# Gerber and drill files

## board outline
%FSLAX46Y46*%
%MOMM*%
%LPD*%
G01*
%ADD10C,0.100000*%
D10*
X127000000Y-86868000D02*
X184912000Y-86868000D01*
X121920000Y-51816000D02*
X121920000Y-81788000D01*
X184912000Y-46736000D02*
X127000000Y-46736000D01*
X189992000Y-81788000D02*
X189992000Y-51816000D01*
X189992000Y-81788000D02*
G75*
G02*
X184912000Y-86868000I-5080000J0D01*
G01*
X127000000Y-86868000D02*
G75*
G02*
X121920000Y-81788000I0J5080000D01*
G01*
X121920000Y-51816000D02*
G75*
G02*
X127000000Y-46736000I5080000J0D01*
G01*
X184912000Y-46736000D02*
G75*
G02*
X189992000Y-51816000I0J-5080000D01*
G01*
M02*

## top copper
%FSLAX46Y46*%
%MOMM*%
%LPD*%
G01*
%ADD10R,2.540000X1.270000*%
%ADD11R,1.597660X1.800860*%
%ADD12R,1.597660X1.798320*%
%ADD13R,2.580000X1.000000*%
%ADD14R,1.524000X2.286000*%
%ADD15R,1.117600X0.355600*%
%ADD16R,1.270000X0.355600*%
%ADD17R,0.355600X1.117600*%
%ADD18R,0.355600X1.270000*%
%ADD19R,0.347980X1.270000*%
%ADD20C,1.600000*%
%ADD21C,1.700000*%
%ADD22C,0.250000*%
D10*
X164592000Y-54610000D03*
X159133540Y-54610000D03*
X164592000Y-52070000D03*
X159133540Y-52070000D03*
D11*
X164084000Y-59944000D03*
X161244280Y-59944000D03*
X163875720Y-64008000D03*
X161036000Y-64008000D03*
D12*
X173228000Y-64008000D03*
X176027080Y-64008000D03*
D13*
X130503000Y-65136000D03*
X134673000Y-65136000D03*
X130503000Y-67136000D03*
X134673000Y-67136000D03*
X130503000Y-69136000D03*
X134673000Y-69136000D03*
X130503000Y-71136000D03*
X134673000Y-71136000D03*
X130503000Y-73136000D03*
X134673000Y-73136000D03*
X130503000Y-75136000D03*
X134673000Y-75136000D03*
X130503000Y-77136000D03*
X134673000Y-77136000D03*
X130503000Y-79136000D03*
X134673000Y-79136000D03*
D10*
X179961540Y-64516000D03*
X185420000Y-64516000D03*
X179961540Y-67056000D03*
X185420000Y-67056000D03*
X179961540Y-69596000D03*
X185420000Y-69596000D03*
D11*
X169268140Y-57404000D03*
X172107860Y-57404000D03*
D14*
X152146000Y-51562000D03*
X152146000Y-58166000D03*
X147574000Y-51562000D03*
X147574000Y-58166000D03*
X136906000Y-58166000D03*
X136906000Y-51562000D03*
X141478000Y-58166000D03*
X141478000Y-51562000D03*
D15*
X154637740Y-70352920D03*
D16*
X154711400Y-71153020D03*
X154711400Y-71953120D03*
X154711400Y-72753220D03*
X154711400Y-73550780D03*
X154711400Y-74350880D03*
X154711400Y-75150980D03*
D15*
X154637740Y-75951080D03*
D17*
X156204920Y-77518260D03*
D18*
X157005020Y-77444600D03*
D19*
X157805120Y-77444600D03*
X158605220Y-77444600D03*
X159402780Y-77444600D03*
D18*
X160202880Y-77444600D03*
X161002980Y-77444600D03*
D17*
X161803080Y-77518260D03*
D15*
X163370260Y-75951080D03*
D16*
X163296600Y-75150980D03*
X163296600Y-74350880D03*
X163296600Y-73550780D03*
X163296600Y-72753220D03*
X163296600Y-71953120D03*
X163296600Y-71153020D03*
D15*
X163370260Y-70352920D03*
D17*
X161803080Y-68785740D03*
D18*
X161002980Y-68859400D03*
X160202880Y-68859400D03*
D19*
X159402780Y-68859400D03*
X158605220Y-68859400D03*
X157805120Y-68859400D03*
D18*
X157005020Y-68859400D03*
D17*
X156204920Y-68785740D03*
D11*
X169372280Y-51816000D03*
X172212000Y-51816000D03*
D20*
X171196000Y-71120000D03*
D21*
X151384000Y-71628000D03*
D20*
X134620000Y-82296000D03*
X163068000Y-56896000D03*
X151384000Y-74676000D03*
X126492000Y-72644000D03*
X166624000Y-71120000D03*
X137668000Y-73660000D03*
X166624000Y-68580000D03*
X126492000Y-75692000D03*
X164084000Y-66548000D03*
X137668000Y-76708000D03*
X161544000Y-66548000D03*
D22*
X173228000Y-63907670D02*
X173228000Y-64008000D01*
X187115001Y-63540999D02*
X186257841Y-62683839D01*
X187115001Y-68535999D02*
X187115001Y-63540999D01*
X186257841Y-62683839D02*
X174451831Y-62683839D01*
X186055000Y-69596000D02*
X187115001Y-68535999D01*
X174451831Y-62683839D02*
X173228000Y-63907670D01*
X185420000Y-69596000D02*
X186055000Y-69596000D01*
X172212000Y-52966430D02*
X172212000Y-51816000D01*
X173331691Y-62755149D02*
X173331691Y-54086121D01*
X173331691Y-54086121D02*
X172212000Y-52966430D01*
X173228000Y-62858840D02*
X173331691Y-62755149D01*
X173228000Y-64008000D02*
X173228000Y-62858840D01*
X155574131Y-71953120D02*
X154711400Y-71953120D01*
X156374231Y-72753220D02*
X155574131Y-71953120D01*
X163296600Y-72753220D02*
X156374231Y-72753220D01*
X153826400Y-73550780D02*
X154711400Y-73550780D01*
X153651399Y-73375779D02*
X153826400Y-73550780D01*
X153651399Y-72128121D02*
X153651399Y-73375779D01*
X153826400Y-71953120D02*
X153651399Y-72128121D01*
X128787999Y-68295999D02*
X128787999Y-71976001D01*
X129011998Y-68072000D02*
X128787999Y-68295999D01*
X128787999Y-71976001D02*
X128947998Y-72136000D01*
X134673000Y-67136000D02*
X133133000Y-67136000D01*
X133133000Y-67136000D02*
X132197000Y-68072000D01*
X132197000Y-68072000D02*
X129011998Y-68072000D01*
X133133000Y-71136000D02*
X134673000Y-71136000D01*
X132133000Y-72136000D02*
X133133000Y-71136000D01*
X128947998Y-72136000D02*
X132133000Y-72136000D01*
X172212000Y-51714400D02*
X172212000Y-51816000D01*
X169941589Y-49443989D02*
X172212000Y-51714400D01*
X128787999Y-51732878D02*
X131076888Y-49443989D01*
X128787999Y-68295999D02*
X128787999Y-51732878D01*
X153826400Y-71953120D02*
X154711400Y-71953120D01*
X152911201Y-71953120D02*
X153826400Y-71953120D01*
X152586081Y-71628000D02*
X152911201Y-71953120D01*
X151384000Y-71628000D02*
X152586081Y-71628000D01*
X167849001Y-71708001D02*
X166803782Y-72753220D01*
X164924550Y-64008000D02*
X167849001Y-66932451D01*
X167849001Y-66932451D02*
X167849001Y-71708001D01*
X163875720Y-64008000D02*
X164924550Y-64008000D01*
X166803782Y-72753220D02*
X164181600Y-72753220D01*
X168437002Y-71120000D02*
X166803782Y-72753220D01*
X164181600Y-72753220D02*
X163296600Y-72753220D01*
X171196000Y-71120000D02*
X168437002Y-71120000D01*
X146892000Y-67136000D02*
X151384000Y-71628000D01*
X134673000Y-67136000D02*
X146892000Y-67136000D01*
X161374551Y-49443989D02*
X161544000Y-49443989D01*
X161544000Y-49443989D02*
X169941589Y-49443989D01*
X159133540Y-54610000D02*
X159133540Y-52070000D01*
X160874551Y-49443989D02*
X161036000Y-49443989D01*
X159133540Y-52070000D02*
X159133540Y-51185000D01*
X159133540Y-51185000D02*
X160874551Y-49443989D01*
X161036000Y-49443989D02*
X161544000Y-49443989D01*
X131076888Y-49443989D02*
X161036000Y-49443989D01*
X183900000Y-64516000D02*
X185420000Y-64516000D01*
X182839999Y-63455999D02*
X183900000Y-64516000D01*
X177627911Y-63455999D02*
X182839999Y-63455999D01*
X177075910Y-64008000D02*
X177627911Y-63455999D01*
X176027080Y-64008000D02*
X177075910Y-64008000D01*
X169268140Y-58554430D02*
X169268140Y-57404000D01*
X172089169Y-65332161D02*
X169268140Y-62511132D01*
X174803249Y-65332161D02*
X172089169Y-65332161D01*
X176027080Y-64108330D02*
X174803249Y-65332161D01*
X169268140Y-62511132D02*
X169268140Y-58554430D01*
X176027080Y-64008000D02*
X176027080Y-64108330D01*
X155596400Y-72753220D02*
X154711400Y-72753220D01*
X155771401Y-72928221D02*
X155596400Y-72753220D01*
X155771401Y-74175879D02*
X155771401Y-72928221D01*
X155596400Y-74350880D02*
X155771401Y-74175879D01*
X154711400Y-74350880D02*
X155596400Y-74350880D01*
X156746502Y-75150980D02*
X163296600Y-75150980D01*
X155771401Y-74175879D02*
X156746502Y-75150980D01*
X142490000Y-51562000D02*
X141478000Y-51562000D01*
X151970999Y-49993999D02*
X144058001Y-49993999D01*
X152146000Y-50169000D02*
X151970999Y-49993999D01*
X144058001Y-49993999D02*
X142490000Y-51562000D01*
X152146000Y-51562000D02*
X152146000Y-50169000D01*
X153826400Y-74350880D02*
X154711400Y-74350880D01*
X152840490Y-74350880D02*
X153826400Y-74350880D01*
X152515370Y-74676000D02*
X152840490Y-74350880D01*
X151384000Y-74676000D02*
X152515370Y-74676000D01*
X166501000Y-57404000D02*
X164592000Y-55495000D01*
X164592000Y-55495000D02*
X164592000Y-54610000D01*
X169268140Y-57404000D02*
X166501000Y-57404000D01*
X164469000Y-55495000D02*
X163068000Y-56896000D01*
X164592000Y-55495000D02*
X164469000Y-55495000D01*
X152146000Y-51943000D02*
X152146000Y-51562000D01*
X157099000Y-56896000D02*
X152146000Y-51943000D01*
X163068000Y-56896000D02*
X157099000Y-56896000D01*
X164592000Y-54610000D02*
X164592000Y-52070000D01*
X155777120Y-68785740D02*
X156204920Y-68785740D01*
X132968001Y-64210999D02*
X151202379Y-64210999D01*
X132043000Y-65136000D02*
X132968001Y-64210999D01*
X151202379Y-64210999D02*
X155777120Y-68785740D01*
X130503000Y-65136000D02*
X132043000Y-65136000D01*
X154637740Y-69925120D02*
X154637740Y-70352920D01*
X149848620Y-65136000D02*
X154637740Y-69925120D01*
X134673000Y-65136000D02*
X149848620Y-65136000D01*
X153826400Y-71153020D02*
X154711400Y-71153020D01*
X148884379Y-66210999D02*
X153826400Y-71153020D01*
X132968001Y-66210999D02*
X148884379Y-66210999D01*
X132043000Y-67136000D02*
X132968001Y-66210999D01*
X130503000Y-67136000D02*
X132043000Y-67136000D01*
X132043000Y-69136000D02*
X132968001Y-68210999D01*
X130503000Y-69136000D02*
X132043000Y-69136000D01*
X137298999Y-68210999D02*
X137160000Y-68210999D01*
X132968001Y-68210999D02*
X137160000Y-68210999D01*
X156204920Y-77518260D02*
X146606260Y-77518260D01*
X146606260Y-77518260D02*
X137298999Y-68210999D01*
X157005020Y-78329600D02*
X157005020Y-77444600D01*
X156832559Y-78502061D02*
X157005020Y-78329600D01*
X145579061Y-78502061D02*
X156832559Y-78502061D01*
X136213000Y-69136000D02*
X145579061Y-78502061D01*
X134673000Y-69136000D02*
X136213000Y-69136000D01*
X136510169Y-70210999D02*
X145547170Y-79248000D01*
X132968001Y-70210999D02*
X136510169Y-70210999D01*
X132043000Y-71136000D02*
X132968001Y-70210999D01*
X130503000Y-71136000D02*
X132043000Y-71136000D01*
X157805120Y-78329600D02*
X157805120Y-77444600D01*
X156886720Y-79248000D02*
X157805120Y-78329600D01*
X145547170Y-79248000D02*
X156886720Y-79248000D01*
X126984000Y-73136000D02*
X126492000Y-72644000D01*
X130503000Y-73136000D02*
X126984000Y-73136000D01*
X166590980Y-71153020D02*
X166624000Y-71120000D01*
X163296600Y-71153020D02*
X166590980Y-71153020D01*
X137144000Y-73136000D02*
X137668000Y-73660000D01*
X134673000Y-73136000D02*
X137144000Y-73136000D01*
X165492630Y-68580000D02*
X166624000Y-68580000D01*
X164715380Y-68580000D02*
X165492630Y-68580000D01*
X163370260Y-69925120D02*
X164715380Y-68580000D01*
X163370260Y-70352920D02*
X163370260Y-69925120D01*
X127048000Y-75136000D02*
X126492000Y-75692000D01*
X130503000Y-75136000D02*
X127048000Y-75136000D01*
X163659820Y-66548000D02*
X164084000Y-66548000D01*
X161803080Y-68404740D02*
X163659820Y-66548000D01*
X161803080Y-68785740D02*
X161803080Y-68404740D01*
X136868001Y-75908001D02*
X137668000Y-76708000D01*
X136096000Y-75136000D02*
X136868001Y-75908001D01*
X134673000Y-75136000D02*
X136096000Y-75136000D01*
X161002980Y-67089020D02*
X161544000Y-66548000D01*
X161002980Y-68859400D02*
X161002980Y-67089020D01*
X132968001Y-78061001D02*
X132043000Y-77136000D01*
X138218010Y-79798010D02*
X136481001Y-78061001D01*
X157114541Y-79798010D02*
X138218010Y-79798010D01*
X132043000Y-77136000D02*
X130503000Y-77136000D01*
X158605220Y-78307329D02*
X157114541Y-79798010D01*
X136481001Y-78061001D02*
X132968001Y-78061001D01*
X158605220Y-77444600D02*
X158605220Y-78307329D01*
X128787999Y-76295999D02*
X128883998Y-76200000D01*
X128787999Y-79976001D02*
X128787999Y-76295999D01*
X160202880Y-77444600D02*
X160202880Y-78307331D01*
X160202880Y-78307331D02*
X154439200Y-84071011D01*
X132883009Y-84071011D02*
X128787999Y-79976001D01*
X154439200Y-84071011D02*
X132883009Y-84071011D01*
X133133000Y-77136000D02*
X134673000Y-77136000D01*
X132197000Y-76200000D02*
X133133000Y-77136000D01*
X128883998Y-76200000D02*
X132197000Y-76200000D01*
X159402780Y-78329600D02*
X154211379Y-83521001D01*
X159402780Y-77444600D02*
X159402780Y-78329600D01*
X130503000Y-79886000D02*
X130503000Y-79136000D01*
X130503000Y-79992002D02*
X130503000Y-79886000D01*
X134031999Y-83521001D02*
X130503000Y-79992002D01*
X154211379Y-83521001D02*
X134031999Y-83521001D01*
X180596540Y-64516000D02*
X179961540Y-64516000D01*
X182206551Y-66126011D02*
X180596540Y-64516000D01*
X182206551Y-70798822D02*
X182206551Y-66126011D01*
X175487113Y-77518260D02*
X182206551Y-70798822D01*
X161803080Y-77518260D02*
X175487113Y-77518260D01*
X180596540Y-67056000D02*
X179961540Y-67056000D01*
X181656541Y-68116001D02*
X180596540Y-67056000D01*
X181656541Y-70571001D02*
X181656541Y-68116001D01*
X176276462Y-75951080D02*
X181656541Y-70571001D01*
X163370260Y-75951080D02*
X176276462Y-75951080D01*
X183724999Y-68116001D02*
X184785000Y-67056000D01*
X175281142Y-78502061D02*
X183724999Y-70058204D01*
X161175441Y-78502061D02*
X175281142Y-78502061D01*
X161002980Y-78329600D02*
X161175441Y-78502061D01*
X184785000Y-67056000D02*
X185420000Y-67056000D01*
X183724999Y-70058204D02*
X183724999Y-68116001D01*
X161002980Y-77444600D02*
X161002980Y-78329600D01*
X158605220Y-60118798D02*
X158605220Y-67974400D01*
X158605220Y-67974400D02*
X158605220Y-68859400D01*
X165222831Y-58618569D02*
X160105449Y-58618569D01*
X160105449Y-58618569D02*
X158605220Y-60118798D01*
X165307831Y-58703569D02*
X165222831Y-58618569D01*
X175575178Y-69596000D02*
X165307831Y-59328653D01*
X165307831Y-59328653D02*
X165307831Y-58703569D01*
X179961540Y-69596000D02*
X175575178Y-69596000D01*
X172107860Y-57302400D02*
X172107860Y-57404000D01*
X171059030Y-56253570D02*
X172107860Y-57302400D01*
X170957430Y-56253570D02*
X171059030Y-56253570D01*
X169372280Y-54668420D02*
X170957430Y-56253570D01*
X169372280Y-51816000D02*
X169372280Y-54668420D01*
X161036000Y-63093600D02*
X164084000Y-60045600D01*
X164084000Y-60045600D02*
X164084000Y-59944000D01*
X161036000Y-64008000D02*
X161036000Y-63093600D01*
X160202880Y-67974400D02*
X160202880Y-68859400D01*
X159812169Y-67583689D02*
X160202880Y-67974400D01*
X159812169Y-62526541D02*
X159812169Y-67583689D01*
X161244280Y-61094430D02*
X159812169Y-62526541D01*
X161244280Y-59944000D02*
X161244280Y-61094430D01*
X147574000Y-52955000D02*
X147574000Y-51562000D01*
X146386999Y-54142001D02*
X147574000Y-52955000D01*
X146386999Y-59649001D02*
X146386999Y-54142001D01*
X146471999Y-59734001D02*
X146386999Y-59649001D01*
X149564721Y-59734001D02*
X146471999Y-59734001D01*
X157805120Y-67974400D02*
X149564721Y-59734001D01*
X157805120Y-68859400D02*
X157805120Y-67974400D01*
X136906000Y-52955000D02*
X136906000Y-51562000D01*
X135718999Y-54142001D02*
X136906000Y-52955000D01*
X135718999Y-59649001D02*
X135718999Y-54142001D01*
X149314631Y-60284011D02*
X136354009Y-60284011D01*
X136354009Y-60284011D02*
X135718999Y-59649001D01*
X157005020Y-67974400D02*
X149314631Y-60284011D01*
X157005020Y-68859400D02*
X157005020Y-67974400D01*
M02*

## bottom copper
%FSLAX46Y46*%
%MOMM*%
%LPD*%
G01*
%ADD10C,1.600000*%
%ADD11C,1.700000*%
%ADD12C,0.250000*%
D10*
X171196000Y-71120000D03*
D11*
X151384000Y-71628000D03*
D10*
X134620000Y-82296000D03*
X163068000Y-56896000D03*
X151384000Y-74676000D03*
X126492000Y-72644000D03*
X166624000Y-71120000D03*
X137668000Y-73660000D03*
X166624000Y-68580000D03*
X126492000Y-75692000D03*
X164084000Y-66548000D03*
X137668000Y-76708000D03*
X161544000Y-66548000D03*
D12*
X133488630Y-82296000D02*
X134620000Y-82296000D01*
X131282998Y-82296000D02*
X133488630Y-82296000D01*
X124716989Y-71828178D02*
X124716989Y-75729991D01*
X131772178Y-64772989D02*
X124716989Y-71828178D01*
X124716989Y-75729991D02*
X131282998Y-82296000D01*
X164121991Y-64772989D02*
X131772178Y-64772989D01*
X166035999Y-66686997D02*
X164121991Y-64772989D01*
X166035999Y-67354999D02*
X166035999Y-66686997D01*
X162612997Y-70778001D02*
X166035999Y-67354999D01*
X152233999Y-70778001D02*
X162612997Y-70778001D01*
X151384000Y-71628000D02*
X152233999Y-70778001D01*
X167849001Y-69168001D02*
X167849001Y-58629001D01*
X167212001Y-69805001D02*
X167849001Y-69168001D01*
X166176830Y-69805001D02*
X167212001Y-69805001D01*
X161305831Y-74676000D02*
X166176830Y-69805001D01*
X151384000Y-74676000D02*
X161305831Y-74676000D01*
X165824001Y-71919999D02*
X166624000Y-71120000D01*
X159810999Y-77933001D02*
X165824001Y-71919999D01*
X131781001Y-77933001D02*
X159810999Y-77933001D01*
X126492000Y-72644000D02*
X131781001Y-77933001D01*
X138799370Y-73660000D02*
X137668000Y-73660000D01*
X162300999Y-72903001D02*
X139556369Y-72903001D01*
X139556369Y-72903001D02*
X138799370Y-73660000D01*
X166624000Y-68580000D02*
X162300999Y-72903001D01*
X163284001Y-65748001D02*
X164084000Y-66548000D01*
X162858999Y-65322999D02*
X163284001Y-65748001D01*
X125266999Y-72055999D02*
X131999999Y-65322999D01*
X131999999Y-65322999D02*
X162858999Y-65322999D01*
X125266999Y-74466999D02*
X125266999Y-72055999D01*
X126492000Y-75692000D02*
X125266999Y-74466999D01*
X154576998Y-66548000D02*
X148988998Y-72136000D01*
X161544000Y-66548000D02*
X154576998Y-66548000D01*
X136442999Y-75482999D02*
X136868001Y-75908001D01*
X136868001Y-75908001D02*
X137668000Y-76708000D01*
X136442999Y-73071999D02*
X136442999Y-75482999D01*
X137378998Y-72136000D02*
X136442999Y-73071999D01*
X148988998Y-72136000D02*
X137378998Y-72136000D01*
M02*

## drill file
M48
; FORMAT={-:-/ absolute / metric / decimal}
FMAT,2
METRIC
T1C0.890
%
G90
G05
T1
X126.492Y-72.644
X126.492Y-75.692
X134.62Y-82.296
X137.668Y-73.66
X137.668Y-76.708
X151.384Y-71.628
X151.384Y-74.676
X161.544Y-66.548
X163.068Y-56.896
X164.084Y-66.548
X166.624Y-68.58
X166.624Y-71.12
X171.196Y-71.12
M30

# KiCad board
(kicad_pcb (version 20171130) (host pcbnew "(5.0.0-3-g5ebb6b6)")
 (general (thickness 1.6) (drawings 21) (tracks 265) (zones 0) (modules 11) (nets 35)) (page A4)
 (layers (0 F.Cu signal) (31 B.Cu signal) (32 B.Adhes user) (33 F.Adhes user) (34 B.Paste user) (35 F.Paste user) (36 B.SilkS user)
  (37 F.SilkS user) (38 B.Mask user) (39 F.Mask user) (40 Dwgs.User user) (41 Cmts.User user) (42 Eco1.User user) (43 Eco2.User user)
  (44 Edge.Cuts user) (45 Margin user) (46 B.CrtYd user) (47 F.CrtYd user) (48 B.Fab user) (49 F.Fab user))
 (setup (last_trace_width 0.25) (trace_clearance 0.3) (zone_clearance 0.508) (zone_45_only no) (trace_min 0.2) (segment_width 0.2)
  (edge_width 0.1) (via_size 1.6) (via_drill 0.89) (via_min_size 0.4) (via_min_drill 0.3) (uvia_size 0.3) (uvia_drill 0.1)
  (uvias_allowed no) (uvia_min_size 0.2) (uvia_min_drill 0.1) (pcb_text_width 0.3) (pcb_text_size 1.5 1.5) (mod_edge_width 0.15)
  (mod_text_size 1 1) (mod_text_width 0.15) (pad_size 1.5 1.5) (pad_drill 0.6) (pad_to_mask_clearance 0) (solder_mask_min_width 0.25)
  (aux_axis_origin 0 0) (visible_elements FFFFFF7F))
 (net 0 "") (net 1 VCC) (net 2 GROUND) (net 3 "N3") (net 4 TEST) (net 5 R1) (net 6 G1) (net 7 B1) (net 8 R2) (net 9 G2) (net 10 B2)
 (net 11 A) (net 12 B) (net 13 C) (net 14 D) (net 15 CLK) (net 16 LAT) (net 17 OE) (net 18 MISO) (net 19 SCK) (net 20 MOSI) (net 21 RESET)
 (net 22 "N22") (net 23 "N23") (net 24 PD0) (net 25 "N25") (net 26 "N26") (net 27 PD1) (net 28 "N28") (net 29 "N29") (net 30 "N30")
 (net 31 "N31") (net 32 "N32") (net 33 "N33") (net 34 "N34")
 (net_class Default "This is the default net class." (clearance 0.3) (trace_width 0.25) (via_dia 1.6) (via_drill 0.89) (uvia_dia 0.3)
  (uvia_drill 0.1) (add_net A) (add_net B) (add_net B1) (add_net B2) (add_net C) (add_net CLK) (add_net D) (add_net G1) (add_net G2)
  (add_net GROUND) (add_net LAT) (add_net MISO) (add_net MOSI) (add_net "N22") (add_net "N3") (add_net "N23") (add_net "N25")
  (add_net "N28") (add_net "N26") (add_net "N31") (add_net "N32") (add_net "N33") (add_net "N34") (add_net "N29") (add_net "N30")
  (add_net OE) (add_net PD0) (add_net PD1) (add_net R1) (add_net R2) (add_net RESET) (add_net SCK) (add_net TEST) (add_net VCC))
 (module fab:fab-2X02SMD (layer F.Cu) (at 162.052 53.34 180)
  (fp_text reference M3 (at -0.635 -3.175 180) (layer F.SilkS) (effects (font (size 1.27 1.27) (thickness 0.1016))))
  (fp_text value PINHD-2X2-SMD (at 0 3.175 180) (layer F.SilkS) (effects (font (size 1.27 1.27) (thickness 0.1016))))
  (pad 1 smd rect (at -2.54 -1.27 180) (size 2.54 1.27) (layers F.Cu F.Paste F.Mask) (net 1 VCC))
  (pad 2 smd rect (at 2.91846 -1.27 180) (size 2.54 1.27) (layers F.Cu F.Paste F.Mask) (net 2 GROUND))
  (pad 3 smd rect (at -2.54 1.27 180) (size 2.54 1.27) (layers F.Cu F.Paste F.Mask) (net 1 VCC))
  (pad 4 smd rect (at 2.91846 1.27 180) (size 2.54 1.27) (layers F.Cu F.Paste F.Mask) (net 2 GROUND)))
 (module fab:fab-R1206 (layer F.Cu) (at 162.66414 59.944)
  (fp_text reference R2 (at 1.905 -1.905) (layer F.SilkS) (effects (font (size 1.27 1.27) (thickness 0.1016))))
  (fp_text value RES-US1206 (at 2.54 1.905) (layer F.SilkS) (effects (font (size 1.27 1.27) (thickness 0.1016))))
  (pad 2 smd rect (at 1.41986 0) (size 1.59766 1.80086) (layers F.Cu F.Paste F.Mask) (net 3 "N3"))
  (pad 1 smd rect (at -1.41986 0) (size 1.59766 1.80086) (layers F.Cu F.Paste F.Mask) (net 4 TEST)))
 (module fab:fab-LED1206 (layer F.Cu) (at 162.45586 64.008)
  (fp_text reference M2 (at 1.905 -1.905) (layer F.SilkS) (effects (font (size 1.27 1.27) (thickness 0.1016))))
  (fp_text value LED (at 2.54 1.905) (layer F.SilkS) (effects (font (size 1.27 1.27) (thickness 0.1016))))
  (pad 2 smd rect (at 1.41986 0) (size 1.59766 1.80086) (layers F.Cu F.Paste F.Mask) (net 2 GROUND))
  (pad 1 smd rect (at -1.41986 0) (size 1.59766 1.80086) (layers F.Cu F.Paste F.Mask) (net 3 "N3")))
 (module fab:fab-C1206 (layer F.Cu) (at 174.62754 64.008)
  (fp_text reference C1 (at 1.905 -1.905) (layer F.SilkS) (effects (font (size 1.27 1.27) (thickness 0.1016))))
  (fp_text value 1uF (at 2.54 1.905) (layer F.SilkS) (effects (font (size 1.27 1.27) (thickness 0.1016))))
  (pad 1 smd rect (at -1.39954 0) (size 1.59766 1.79832) (layers F.Cu F.Paste F.Mask) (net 2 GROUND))
  (pad 2 smd rect (at 1.39954 0) (size 1.59766 1.79832) (layers F.Cu F.Paste F.Mask) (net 1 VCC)))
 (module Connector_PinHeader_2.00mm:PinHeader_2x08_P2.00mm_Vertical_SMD (layer F.Cu) (at 132.588 72.136)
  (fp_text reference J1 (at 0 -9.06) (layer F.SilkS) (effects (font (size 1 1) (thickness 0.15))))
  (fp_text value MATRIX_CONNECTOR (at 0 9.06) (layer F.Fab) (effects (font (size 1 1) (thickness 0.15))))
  (pad 1 smd rect (at -2.085 -7) (size 2.58 1) (layers F.Cu F.Paste F.Mask) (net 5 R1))
  (pad 2 smd rect (at 2.085 -7) (size 2.58 1) (layers F.Cu F.Paste F.Mask) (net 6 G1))
  (pad 3 smd rect (at -2.085 -5) (size 2.58 1) (layers F.Cu F.Paste F.Mask) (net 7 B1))
  (pad 4 smd rect (at 2.085 -5) (size 2.58 1) (layers F.Cu F.Paste F.Mask) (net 2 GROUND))
  (pad 5 smd rect (at -2.085 -3) (size 2.58 1) (layers F.Cu F.Paste F.Mask) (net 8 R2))
  (pad 6 smd rect (at 2.085 -3) (size 2.58 1) (layers F.Cu F.Paste F.Mask) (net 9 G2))
  (pad 7 smd rect (at -2.085 -1) (size 2.58 1) (layers F.Cu F.Paste F.Mask) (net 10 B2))
  (pad 8 smd rect (at 2.085 -1) (size 2.58 1) (layers F.Cu F.Paste F.Mask) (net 2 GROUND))
  (pad 9 smd rect (at -2.085 1) (size 2.58 1) (layers F.Cu F.Paste F.Mask) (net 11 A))
  (pad 10 smd rect (at 2.085 1) (size 2.58 1) (layers F.Cu F.Paste F.Mask) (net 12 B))
  (pad 11 smd rect (at -2.085 3) (size 2.58 1) (layers F.Cu F.Paste F.Mask) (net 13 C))
  (pad 12 smd rect (at 2.085 3) (size 2.58 1) (layers F.Cu F.Paste F.Mask) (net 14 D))
  (pad 13 smd rect (at -2.085 5) (size 2.58 1) (layers F.Cu F.Paste F.Mask) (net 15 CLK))
  (pad 14 smd rect (at 2.085 5) (size 2.58 1) (layers F.Cu F.Paste F.Mask) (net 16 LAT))
  (pad 15 smd rect (at -2.085 7) (size 2.58 1) (layers F.Cu F.Paste F.Mask) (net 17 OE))
  (pad 16 smd rect (at 2.085 7) (size 2.58 1) (layers F.Cu F.Paste F.Mask) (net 2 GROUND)))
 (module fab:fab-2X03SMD (layer F.Cu) (at 182.50154 67.056)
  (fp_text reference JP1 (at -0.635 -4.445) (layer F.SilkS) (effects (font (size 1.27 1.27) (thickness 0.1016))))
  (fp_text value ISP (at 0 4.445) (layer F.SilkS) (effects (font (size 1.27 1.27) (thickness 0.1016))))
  (pad 1 smd rect (at -2.54 -2.54) (size 2.54 1.27) (layers F.Cu F.Paste F.Mask) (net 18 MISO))
  (pad 2 smd rect (at 2.91846 -2.54) (size 2.54 1.27) (layers F.Cu F.Paste F.Mask) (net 1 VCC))
  (pad 3 smd rect (at -2.54 0) (size 2.54 1.27) (layers F.Cu F.Paste F.Mask) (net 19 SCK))
  (pad 4 smd rect (at 2.91846 0) (size 2.54 1.27) (layers F.Cu F.Paste F.Mask) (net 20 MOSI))
  (pad 5 smd rect (at -2.54 2.54) (size 2.54 1.27) (layers F.Cu F.Paste F.Mask) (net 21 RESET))
  (pad 6 smd rect (at 2.91846 2.54) (size 2.54 1.27) (layers F.Cu F.Paste F.Mask) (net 2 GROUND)))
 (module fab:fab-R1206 (layer F.Cu) (at 170.688 57.404)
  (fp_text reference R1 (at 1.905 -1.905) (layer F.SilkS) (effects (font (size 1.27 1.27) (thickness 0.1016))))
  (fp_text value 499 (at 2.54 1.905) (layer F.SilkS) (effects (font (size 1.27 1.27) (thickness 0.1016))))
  (pad 1 smd rect (at -1.41986 0) (size 1.59766 1.80086) (layers F.Cu F.Paste F.Mask) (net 1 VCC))
  (pad 2 smd rect (at 1.41986 0) (size 1.59766 1.80086) (layers F.Cu F.Paste F.Mask) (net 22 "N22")))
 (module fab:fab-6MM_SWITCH (layer F.Cu) (at 149.86 54.864 270)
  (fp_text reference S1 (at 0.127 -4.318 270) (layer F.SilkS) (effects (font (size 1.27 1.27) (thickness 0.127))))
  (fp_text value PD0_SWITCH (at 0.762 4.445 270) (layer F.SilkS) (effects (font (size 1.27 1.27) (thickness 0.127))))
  (pad 1 smd rect (at -3.302 -2.286 270) (size 2.286 1.524) (layers F.Cu F.Paste F.Mask) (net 1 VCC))
  (pad 2 smd rect (at 3.302 -2.286 270) (size 2.286 1.524) (layers F.Cu F.Paste F.Mask) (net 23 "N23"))
  (pad 3 smd rect (at -3.302 2.286 270) (size 2.286 1.524) (layers F.Cu F.Paste F.Mask) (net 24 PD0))
  (pad 4 smd rect (at 3.302 2.286 270) (size 2.286 1.524) (layers F.Cu F.Paste F.Mask) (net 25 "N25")))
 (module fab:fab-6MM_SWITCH (layer F.Cu) (at 139.192 54.864 270)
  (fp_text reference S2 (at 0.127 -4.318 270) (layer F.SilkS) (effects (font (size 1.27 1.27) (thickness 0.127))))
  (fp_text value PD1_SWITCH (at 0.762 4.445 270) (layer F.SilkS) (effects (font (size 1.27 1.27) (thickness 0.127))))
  (pad 4 smd rect (at 3.302 2.286 270) (size 2.286 1.524) (layers F.Cu F.Paste F.Mask) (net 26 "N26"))
  (pad 3 smd rect (at -3.302 2.286 270) (size 2.286 1.524) (layers F.Cu F.Paste F.Mask) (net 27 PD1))
  (pad 2 smd rect (at 3.302 -2.286 270) (size 2.286 1.524) (layers F.Cu F.Paste F.Mask) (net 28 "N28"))
  (pad 1 smd rect (at -3.302 -2.286 270) (size 2.286 1.524) (layers F.Cu F.Paste F.Mask) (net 1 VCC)))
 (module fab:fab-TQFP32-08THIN (layer F.Cu) (at 159.004 73.152)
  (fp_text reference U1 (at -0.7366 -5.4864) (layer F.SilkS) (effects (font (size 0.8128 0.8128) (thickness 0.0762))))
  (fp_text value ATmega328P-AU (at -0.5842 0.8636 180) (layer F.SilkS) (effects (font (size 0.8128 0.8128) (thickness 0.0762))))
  (pad 1 smd rect (at -4.36626 -2.79908) (size 1.1176 0.3556) (layers F.Cu F.Paste F.Mask) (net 6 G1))
  (pad 2 smd rect (at -4.2926 -1.99898) (size 1.27 0.3556) (layers F.Cu F.Paste F.Mask) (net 7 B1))
  (pad 3 smd rect (at -4.2926 -1.19888) (size 1.27 0.3556) (layers F.Cu F.Paste F.Mask) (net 2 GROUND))
  (pad 4 smd rect (at -4.2926 -0.39878) (size 1.27 0.3556) (layers F.Cu F.Paste F.Mask) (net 1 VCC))
  (pad 5 smd rect (at -4.2926 0.39878) (size 1.27 0.3556) (layers F.Cu F.Paste F.Mask) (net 2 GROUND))
  (pad 6 smd rect (at -4.2926 1.19888) (size 1.27 0.3556) (layers F.Cu F.Paste F.Mask) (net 1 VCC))
  (pad 7 smd rect (at -4.2926 1.99898) (size 1.27 0.3556) (layers F.Cu F.Paste F.Mask) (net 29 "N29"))
  (pad 8 smd rect (at -4.36626 2.79908) (size 1.1176 0.3556) (layers F.Cu F.Paste F.Mask) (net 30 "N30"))
  (pad 9 smd rect (at -2.79908 4.36626) (size 0.3556 1.1176) (layers F.Cu F.Paste F.Mask) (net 8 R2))
  (pad 10 smd rect (at -1.99898 4.2926) (size 0.3556 1.27) (layers F.Cu F.Paste F.Mask) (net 9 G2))
  (pad 11 smd rect (at -1.19888 4.2926) (size 0.34798 1.27) (layers F.Cu F.Paste F.Mask) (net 10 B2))
  (pad 12 smd rect (at -0.39878 4.2926) (size 0.34798 1.27) (layers F.Cu F.Paste F.Mask) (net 15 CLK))
  (pad 13 smd rect (at 0.39878 4.2926) (size 0.34798 1.27) (layers F.Cu F.Paste F.Mask) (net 17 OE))
  (pad 14 smd rect (at 1.19888 4.2926) (size 0.3556 1.27) (layers F.Cu F.Paste F.Mask) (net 16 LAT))
  (pad 15 smd rect (at 1.99898 4.2926) (size 0.3556 1.27) (layers F.Cu F.Paste F.Mask) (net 20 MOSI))
  (pad 16 smd rect (at 2.79908 4.36626) (size 0.3556 1.1176) (layers F.Cu F.Paste F.Mask) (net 18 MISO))
  (pad 17 smd rect (at 4.36626 2.79908) (size 1.1176 0.3556) (layers F.Cu F.Paste F.Mask) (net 19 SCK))
  (pad 18 smd rect (at 4.2926 1.99898) (size 1.27 0.3556) (layers F.Cu F.Paste F.Mask) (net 1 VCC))
  (pad 19 smd rect (at 4.2926 1.19888) (size 1.27 0.3556) (layers F.Cu F.Paste F.Mask) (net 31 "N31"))
  (pad 20 smd rect (at 4.2926 0.39878) (size 1.27 0.3556) (layers F.Cu F.Paste F.Mask) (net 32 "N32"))
  (pad 21 smd rect (at 4.2926 -0.39878) (size 1.27 0.3556) (layers F.Cu F.Paste F.Mask) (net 2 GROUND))
  (pad 22 smd rect (at 4.2926 -1.19888) (size 1.27 0.3556) (layers F.Cu F.Paste F.Mask) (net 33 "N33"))
  (pad 23 smd rect (at 4.2926 -1.99898) (size 1.27 0.3556) (layers F.Cu F.Paste F.Mask) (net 11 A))
  (pad 24 smd rect (at 4.36626 -2.79908) (size 1.1176 0.3556) (layers F.Cu F.Paste F.Mask) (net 12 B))
  (pad 25 smd rect (at 2.79908 -4.36626) (size 0.3556 1.1176) (layers F.Cu F.Paste F.Mask) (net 13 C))
  (pad 26 smd rect (at 1.99898 -4.2926) (size 0.3556 1.27) (layers F.Cu F.Paste F.Mask) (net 14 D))
  (pad 27 smd rect (at 1.19888 -4.2926) (size 0.3556 1.27) (layers F.Cu F.Paste F.Mask) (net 4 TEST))
  (pad 28 smd rect (at 0.39878 -4.2926) (size 0.34798 1.27) (layers F.Cu F.Paste F.Mask) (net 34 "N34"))
  (pad 29 smd rect (at -0.39878 -4.2926) (size 0.34798 1.27) (layers F.Cu F.Paste F.Mask) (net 21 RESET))
  (pad 30 smd rect (at -1.19888 -4.2926) (size 0.34798 1.27) (layers F.Cu F.Paste F.Mask) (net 24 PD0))
  (pad 31 smd rect (at -1.99898 -4.2926) (size 0.3556 1.27) (layers F.Cu F.Paste F.Mask) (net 27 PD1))
  (pad 32 smd rect (at -2.79908 -4.36626) (size 0.3556 1.1176) (layers F.Cu F.Paste F.Mask) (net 5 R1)))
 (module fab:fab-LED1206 (layer F.Cu) (at 170.79214 51.816)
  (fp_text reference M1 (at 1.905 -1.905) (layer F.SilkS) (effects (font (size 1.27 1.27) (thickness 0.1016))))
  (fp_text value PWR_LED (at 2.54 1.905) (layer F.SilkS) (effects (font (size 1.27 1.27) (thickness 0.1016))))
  (pad 1 smd rect (at -1.41986 0) (size 1.59766 1.80086) (layers F.Cu F.Paste F.Mask) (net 22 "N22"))
  (pad 2 smd rect (at 1.41986 0) (size 1.59766 1.80086) (layers F.Cu F.Paste F.Mask) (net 2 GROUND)))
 (gr_line (start 127 86.868) (end 184.912 86.868) (layer Edge.Cuts) (width 0.1))
 (gr_line (start 121.92 51.816) (end 121.92 81.788) (layer Edge.Cuts) (width 0.1))
 (gr_line (start 184.912 46.736) (end 127 46.736) (layer Edge.Cuts) (width 0.1))
 (gr_line (start 189.992 81.788) (end 189.992 51.816) (layer Edge.Cuts) (width 0.1))
 (gr_arc (start 184.912 81.788) (end 184.912 86.868) (angle -90) (layer Edge.Cuts) (width 0.1))
 (gr_arc (start 127 81.788) (end 121.92 81.788) (angle -90) (layer Edge.Cuts) (width 0.1))
 (gr_arc (start 127 51.816) (end 127 46.736) (angle -90) (layer Edge.Cuts) (width 0.1))
 (gr_arc (start 184.912 51.816) (end 189.992 51.816) (angle -90) (layer Edge.Cuts) (width 0.1))
 (via (at 171.196 71.12) (size 1.6) (drill 0.89) (layers F.Cu B.Cu) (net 2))
 (via (at 151.384 71.628) (size 1.7) (drill 0.89) (layers F.Cu B.Cu) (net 2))
 (via (at 134.62 82.296) (size 1.6) (drill 0.89) (layers F.Cu B.Cu) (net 2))
 (segment (start 173.228 63.90767) (end 173.228 64.008) (width 0.25) (layer F.Cu) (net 2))
 (segment (start 187.115001 63.540999) (end 186.257841 62.683839) (width 0.25) (layer F.Cu) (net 2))
 (segment (start 187.115001 68.535999) (end 187.115001 63.540999) (width 0.25) (layer F.Cu) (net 2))
 (segment (start 186.257841 62.683839) (end 174.451831 62.683839) (width 0.25) (layer F.Cu) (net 2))
 (segment (start 186.055 69.596) (end 187.115001 68.535999) (width 0.25) (layer F.Cu) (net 2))
 (segment (start 174.451831 62.683839) (end 173.228 63.90767) (width 0.25) (layer F.Cu) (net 2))
 (segment (start 185.42 69.596) (end 186.055 69.596) (width 0.25) (layer F.Cu) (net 2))
 (segment (start 172.212 52.96643) (end 172.212 51.816) (width 0.25) (layer F.Cu) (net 2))
 (segment (start 173.331691 62.755149) (end 173.331691 54.086121) (width 0.25) (layer F.Cu) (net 2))
 (segment (start 173.331691 54.086121) (end 172.212 52.96643) (width 0.25) (layer F.Cu) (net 2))
 (segment (start 173.228 62.85884) (end 173.331691 62.755149) (width 0.25) (layer F.Cu) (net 2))
 (segment (start 173.228 64.008) (end 173.228 62.85884) (width 0.25) (layer F.Cu) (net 2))
 (segment (start 155.574131 71.95312) (end 154.7114 71.95312) (width 0.25) (layer F.Cu) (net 2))
 (segment (start 156.374231 72.75322) (end 155.574131 71.95312) (width 0.25) (layer F.Cu) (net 2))
 (segment (start 163.2966 72.75322) (end 156.374231 72.75322) (width 0.25) (layer F.Cu) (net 2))
 (segment (start 153.8264 73.55078) (end 154.7114 73.55078) (width 0.25) (layer F.Cu) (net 2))
 (segment (start 153.651399 73.375779) (end 153.8264 73.55078) (width 0.25) (layer F.Cu) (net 2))
 (segment (start 153.651399 72.128121) (end 153.651399 73.375779) (width 0.25) (layer F.Cu) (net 2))
 (segment (start 153.8264 71.95312) (end 153.651399 72.128121) (width 0.25) (layer F.Cu) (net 2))
 (segment (start 128.787999 68.295999) (end 128.787999 71.976001) (width 0.25) (layer F.Cu) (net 2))
 (segment (start 129.011998 68.072) (end 128.787999 68.295999) (width 0.25) (layer F.Cu) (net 2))
 (segment (start 128.787999 71.976001) (end 128.947998 72.136) (width 0.25) (layer F.Cu) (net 2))
 (segment (start 134.673 67.136) (end 133.133 67.136) (width 0.25) (layer F.Cu) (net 2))
 (segment (start 133.133 67.136) (end 132.197 68.072) (width 0.25) (layer F.Cu) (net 2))
 (segment (start 132.197 68.072) (end 129.011998 68.072) (width 0.25) (layer F.Cu) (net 2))
 (segment (start 133.133 71.136) (end 134.673 71.136) (width 0.25) (layer F.Cu) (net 2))
 (segment (start 132.133 72.136) (end 133.133 71.136) (width 0.25) (layer F.Cu) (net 2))
 (segment (start 128.947998 72.136) (end 132.133 72.136) (width 0.25) (layer F.Cu) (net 2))
 (segment (start 172.212 51.7144) (end 172.212 51.816) (width 0.25) (layer F.Cu) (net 2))
 (segment (start 169.941589 49.443989) (end 172.212 51.7144) (width 0.25) (layer F.Cu) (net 2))
 (segment (start 128.787999 51.732878) (end 131.076888 49.443989) (width 0.25) (layer F.Cu) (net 2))
 (segment (start 128.787999 68.295999) (end 128.787999 51.732878) (width 0.25) (layer F.Cu) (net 2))
 (segment (start 153.8264 71.95312) (end 154.7114 71.95312) (width 0.25) (layer F.Cu) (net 2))
 (segment (start 152.911201 71.95312) (end 153.8264 71.95312) (width 0.25) (layer F.Cu) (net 2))
 (segment (start 152.586081 71.628) (end 152.911201 71.95312) (width 0.25) (layer F.Cu) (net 2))
 (segment (start 151.384 71.628) (end 152.586081 71.628) (width 0.25) (layer F.Cu) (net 2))
 (segment (start 167.849001 71.708001) (end 166.803782 72.75322) (width 0.25) (layer F.Cu) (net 2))
 (segment (start 164.92455 64.008) (end 167.849001 66.932451) (width 0.25) (layer F.Cu) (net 2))
 (segment (start 167.849001 66.932451) (end 167.849001 71.708001) (width 0.25) (layer F.Cu) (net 2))
 (segment (start 163.87572 64.008) (end 164.92455 64.008) (width 0.25) (layer F.Cu) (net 2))
 (segment (start 166.803782 72.75322) (end 164.1816 72.75322) (width 0.25) (layer F.Cu) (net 2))
 (segment (start 168.437002 71.12) (end 166.803782 72.75322) (width 0.25) (layer F.Cu) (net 2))
 (segment (start 164.1816 72.75322) (end 163.2966 72.75322) (width 0.25) (layer F.Cu) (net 2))
 (segment (start 171.196 71.12) (end 168.437002 71.12) (width 0.25) (layer F.Cu) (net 2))
 (segment (start 133.48863 82.296) (end 134.62 82.296) (width 0.25) (layer B.Cu) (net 2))
 (segment (start 131.282998 82.296) (end 133.48863 82.296) (width 0.25) (layer B.Cu) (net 2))
 (segment (start 124.716989 71.828178) (end 124.716989 75.729991) (width 0.25) (layer B.Cu) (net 2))
 (segment (start 131.772178 64.772989) (end 124.716989 71.828178) (width 0.25) (layer B.Cu) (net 2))
 (segment (start 124.716989 75.729991) (end 131.282998 82.296) (width 0.25) (layer B.Cu) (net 2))
 (segment (start 164.121991 64.772989) (end 131.772178 64.772989) (width 0.25) (layer B.Cu) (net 2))
 (segment (start 166.035999 66.686997) (end 164.121991 64.772989) (width 0.25) (layer B.Cu) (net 2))
 (segment (start 166.035999 67.354999) (end 166.035999 66.686997) (width 0.25) (layer B.Cu) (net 2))
 (segment (start 162.612997 70.778001) (end 166.035999 67.354999) (width 0.25) (layer B.Cu) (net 2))
 (segment (start 152.233999 70.778001) (end 162.612997 70.778001) (width 0.25) (layer B.Cu) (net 2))
 (segment (start 151.384 71.628) (end 152.233999 70.778001) (width 0.25) (layer B.Cu) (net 2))
 (segment (start 146.892 67.136) (end 151.384 71.628) (width 0.25) (layer F.Cu) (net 2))
 (segment (start 134.673 67.136) (end 146.892 67.136) (width 0.25) (layer F.Cu) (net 2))
 (segment (start 161.374551 49.443989) (end 161.544 49.443989) (width 0.25) (layer F.Cu) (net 2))
 (segment (start 161.544 49.443989) (end 169.941589 49.443989) (width 0.25) (layer F.Cu) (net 2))
 (segment (start 159.13354 54.61) (end 159.13354 52.07) (width 0.25) (layer F.Cu) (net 2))
 (segment (start 160.874551 49.443989) (end 161.036 49.443989) (width 0.25) (layer F.Cu) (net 2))
 (segment (start 159.13354 52.07) (end 159.13354 51.185) (width 0.25) (layer F.Cu) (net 2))
 (segment (start 159.13354 51.185) (end 160.874551 49.443989) (width 0.25) (layer F.Cu) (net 2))
 (segment (start 161.036 49.443989) (end 161.544 49.443989) (width 0.25) (layer F.Cu) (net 2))
 (segment (start 131.076888 49.443989) (end 161.036 49.443989) (width 0.25) (layer F.Cu) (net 2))
 (via (at 163.068 56.896) (size 1.6) (drill 0.89) (layers F.Cu B.Cu) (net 1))
 (via (at 151.384 74.676) (size 1.6) (drill 0.89) (layers F.Cu B.Cu) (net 1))
 (segment (start 183.9 64.516) (end 185.42 64.516) (width 0.25) (layer F.Cu) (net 1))
 (segment (start 182.839999 63.455999) (end 183.9 64.516) (width 0.25) (layer F.Cu) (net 1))
 (segment (start 177.627911 63.455999) (end 182.839999 63.455999) (width 0.25) (layer F.Cu) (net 1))
 (segment (start 177.07591 64.008) (end 177.627911 63.455999) (width 0.25) (layer F.Cu) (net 1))
 (segment (start 176.02708 64.008) (end 177.07591 64.008) (width 0.25) (layer F.Cu) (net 1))
 (segment (start 169.26814 58.55443) (end 169.26814 57.404) (width 0.25) (layer F.Cu) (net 1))
 (segment (start 172.089169 65.332161) (end 169.26814 62.511132) (width 0.25) (layer F.Cu) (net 1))
 (segment (start 174.803249 65.332161) (end 172.089169 65.332161) (width 0.25) (layer F.Cu) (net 1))
 (segment (start 176.02708 64.10833) (end 174.803249 65.332161) (width 0.25) (layer F.Cu) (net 1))
 (segment (start 169.26814 62.511132) (end 169.26814 58.55443) (width 0.25) (layer F.Cu) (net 1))
 (segment (start 176.02708 64.008) (end 176.02708 64.10833) (width 0.25) (layer F.Cu) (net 1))
 (segment (start 155.5964 72.75322) (end 154.7114 72.75322) (width 0.25) (layer F.Cu) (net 1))
 (segment (start 155.771401 72.928221) (end 155.5964 72.75322) (width 0.25) (layer F.Cu) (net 1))
 (segment (start 155.771401 74.175879) (end 155.771401 72.928221) (width 0.25) (layer F.Cu) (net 1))
 (segment (start 155.5964 74.35088) (end 155.771401 74.175879) (width 0.25) (layer F.Cu) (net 1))
 (segment (start 154.7114 74.35088) (end 155.5964 74.35088) (width 0.25) (layer F.Cu) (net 1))
 (segment (start 156.746502 75.15098) (end 163.2966 75.15098) (width 0.25) (layer F.Cu) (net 1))
 (segment (start 155.771401 74.175879) (end 156.746502 75.15098) (width 0.25) (layer F.Cu) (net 1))
 (segment (start 142.49 51.562) (end 141.478 51.562) (width 0.25) (layer F.Cu) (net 1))
 (segment (start 151.970999 49.993999) (end 144.058001 49.993999) (width 0.25) (layer F.Cu) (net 1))
 (segment (start 152.146 50.169) (end 151.970999 49.993999) (width 0.25) (layer F.Cu) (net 1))
 (segment (start 144.058001 49.993999) (end 142.49 51.562) (width 0.25) (layer F.Cu) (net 1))
 (segment (start 152.146 51.562) (end 152.146 50.169) (width 0.25) (layer F.Cu) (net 1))
 (segment (start 153.8264 74.35088) (end 154.7114 74.35088) (width 0.25) (layer F.Cu) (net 1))
 (segment (start 152.84049 74.35088) (end 153.8264 74.35088) (width 0.25) (layer F.Cu) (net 1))
 (segment (start 152.51537 74.676) (end 152.84049 74.35088) (width 0.25) (layer F.Cu) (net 1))
 (segment (start 151.384 74.676) (end 152.51537 74.676) (width 0.25) (layer F.Cu) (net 1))
 (segment (start 167.849001 69.168001) (end 167.849001 58.629001) (width 0.25) (layer B.Cu) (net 1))
 (segment (start 167.212001 69.805001) (end 167.849001 69.168001) (width 0.25) (layer B.Cu) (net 1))
 (segment (start 166.17683 69.805001) (end 167.212001 69.805001) (width 0.25) (layer B.Cu) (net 1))
 (segment (start 161.305831 74.676) (end 166.17683 69.805001) (width 0.25) (layer B.Cu) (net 1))
 (segment (start 151.384 74.676) (end 161.305831 74.676) (width 0.25) (layer B.Cu) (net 1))
 (segment (start 166.501 57.404) (end 164.592 55.495) (width 0.25) (layer F.Cu) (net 1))
 (segment (start 164.592 55.495) (end 164.592 54.61) (width 0.25) (layer F.Cu) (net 1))
 (segment (start 169.26814 57.404) (end 166.501 57.404) (width 0.25) (layer F.Cu) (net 1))
 (segment (start 164.469 55.495) (end 163.068 56.896) (width 0.25) (layer F.Cu) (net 1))
 (segment (start 164.592 55.495) (end 164.469 55.495) (width 0.25) (layer F.Cu) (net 1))
 (segment (start 152.146 51.943) (end 152.146 51.562) (width 0.25) (layer F.Cu) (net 1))
 (segment (start 157.099 56.896) (end 152.146 51.943) (width 0.25) (layer F.Cu) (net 1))
 (segment (start 163.068 56.896) (end 157.099 56.896) (width 0.25) (layer F.Cu) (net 1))
 (segment (start 164.592 54.61) (end 164.592 52.07) (width 0.25) (layer F.Cu) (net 1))
 (segment (start 155.77712 68.78574) (end 156.20492 68.78574) (width 0.25) (layer F.Cu) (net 5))
 (segment (start 132.968001 64.210999) (end 151.202379 64.210999) (width 0.25) (layer F.Cu) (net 5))
 (segment (start 132.043 65.136) (end 132.968001 64.210999) (width 0.25) (layer F.Cu) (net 5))
 (segment (start 151.202379 64.210999) (end 155.77712 68.78574) (width 0.25) (layer F.Cu) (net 5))
 (segment (start 130.503 65.136) (end 132.043 65.136) (width 0.25) (layer F.Cu) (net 5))
 (segment (start 154.63774 69.92512) (end 154.63774 70.35292) (width 0.25) (layer F.Cu) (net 6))
 (segment (start 149.84862 65.136) (end 154.63774 69.92512) (width 0.25) (layer F.Cu) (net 6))
 (segment (start 134.673 65.136) (end 149.84862 65.136) (width 0.25) (layer F.Cu) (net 6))
 (segment (start 153.8264 71.15302) (end 154.7114 71.15302) (width 0.25) (layer F.Cu) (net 7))
 (segment (start 148.884379 66.210999) (end 153.8264 71.15302) (width 0.25) (layer F.Cu) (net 7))
 (segment (start 132.968001 66.210999) (end 148.884379 66.210999) (width 0.25) (layer F.Cu) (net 7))
 (segment (start 132.043 67.136) (end 132.968001 66.210999) (width 0.25) (layer F.Cu) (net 7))
 (segment (start 130.503 67.136) (end 132.043 67.136) (width 0.25) (layer F.Cu) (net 7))
 (segment (start 132.043 69.136) (end 132.968001 68.210999) (width 0.25) (layer F.Cu) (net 8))
 (segment (start 130.503 69.136) (end 132.043 69.136) (width 0.25) (layer F.Cu) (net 8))
 (segment (start 137.298999 68.210999) (end 137.16 68.210999) (width 0.25) (layer F.Cu) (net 8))
 (segment (start 132.968001 68.210999) (end 137.16 68.210999) (width 0.25) (layer F.Cu) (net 8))
 (segment (start 156.20492 77.51826) (end 146.60626 77.51826) (width 0.25) (layer F.Cu) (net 8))
 (segment (start 146.60626 77.51826) (end 137.298999 68.210999) (width 0.25) (layer F.Cu) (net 8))
 (segment (start 157.00502 78.3296) (end 157.00502 77.4446) (width 0.25) (layer F.Cu) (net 9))
 (segment (start 156.832559 78.502061) (end 157.00502 78.3296) (width 0.25) (layer F.Cu) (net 9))
 (segment (start 145.579061 78.502061) (end 156.832559 78.502061) (width 0.25) (layer F.Cu) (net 9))
 (segment (start 136.213 69.136) (end 145.579061 78.502061) (width 0.25) (layer F.Cu) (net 9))
 (segment (start 134.673 69.136) (end 136.213 69.136) (width 0.25) (layer F.Cu) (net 9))
 (segment (start 136.510169 70.210999) (end 145.54717 79.248) (width 0.25) (layer F.Cu) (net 10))
 (segment (start 132.968001 70.210999) (end 136.510169 70.210999) (width 0.25) (layer F.Cu) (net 10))
 (segment (start 132.043 71.136) (end 132.968001 70.210999) (width 0.25) (layer F.Cu) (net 10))
 (segment (start 130.503 71.136) (end 132.043 71.136) (width 0.25) (layer F.Cu) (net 10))
 (segment (start 157.80512 78.3296) (end 157.80512 77.4446) (width 0.25) (layer F.Cu) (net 10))
 (segment (start 156.88672 79.248) (end 157.80512 78.3296) (width 0.25) (layer F.Cu) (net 10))
 (segment (start 145.54717 79.248) (end 156.88672 79.248) (width 0.25) (layer F.Cu) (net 10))
 (via (at 126.492 72.644) (size 1.6) (drill 0.89) (layers F.Cu B.Cu) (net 11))
 (via (at 166.624 71.12) (size 1.6) (drill 0.89) (layers F.Cu B.Cu) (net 11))
 (segment (start 126.984 73.136) (end 126.492 72.644) (width 0.25) (layer F.Cu) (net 11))
 (segment (start 130.503 73.136) (end 126.984 73.136) (width 0.25) (layer F.Cu) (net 11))
 (segment (start 166.59098 71.15302) (end 166.624 71.12) (width 0.25) (layer F.Cu) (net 11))
 (segment (start 163.2966 71.15302) (end 166.59098 71.15302) (width 0.25) (layer F.Cu) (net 11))
 (segment (start 165.824001 71.919999) (end 166.624 71.12) (width 0.25) (layer B.Cu) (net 11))
 (segment (start 159.810999 77.933001) (end 165.824001 71.919999) (width 0.25) (layer B.Cu) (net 11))
 (segment (start 131.781001 77.933001) (end 159.810999 77.933001) (width 0.25) (layer B.Cu) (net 11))
 (segment (start 126.492 72.644) (end 131.781001 77.933001) (width 0.25) (layer B.Cu) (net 11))
 (via (at 137.668 73.66) (size 1.6) (drill 0.89) (layers F.Cu B.Cu) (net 12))
 (via (at 166.624 68.58) (size 1.6) (drill 0.89) (layers F.Cu B.Cu) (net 12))
 (segment (start 137.144 73.136) (end 137.668 73.66) (width 0.25) (layer F.Cu) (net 12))
 (segment (start 134.673 73.136) (end 137.144 73.136) (width 0.25) (layer F.Cu) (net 12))
 (segment (start 165.49263 68.58) (end 166.624 68.58) (width 0.25) (layer F.Cu) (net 12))
 (segment (start 164.71538 68.58) (end 165.49263 68.58) (width 0.25) (layer F.Cu) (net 12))
 (segment (start 163.37026 69.92512) (end 164.71538 68.58) (width 0.25) (layer F.Cu) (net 12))
 (segment (start 163.37026 70.35292) (end 163.37026 69.92512) (width 0.25) (layer F.Cu) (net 12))
 (segment (start 138.79937 73.66) (end 137.668 73.66) (width 0.25) (layer B.Cu) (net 12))
 (segment (start 162.300999 72.903001) (end 139.556369 72.903001) (width 0.25) (layer B.Cu) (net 12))
 (segment (start 139.556369 72.903001) (end 138.79937 73.66) (width 0.25) (layer B.Cu) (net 12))
 (segment (start 166.624 68.58) (end 162.300999 72.903001) (width 0.25) (layer B.Cu) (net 12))
 (via (at 126.492 75.692) (size 1.6) (drill 0.89) (layers F.Cu B.Cu) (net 13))
 (via (at 164.084 66.548) (size 1.6) (drill 0.89) (layers F.Cu B.Cu) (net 13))
 (segment (start 127.048 75.136) (end 126.492 75.692) (width 0.25) (layer F.Cu) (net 13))
 (segment (start 130.503 75.136) (end 127.048 75.136) (width 0.25) (layer F.Cu) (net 13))
 (segment (start 163.65982 66.548) (end 164.084 66.548) (width 0.25) (layer F.Cu) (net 13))
 (segment (start 161.80308 68.40474) (end 163.65982 66.548) (width 0.25) (layer F.Cu) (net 13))
 (segment (start 161.80308 68.78574) (end 161.80308 68.40474) (width 0.25) (layer F.Cu) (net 13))
 (segment (start 163.284001 65.748001) (end 164.084 66.548) (width 0.25) (layer B.Cu) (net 13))
 (segment (start 162.858999 65.322999) (end 163.284001 65.748001) (width 0.25) (layer B.Cu) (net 13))
 (segment (start 125.266999 72.055999) (end 131.999999 65.322999) (width 0.25) (layer B.Cu) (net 13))
 (segment (start 131.999999 65.322999) (end 162.858999 65.322999) (width 0.25) (layer B.Cu) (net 13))
 (segment (start 125.266999 74.466999) (end 125.266999 72.055999) (width 0.25) (layer B.Cu) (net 13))
 (segment (start 126.492 75.692) (end 125.266999 74.466999) (width 0.25) (layer B.Cu) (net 13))
 (via (at 137.668 76.708) (size 1.6) (drill 0.89) (layers F.Cu B.Cu) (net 14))
 (via (at 161.544 66.548) (size 1.6) (drill 0.89) (layers F.Cu B.Cu) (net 14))
 (segment (start 136.868001 75.908001) (end 137.668 76.708) (width 0.25) (layer F.Cu) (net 14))
 (segment (start 136.096 75.136) (end 136.868001 75.908001) (width 0.25) (layer F.Cu) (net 14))
 (segment (start 134.673 75.136) (end 136.096 75.136) (width 0.25) (layer F.Cu) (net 14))
 (segment (start 161.00298 67.08902) (end 161.544 66.548) (width 0.25) (layer F.Cu) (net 14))
 (segment (start 161.00298 68.8594) (end 161.00298 67.08902) (width 0.25) (layer F.Cu) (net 14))
 (segment (start 154.576998 66.548) (end 148.988998 72.136) (width 0.25) (layer B.Cu) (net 14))
 (segment (start 161.544 66.548) (end 154.576998 66.548) (width 0.25) (layer B.Cu) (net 14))
 (segment (start 136.442999 75.482999) (end 136.868001 75.908001) (width 0.25) (layer B.Cu) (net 14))
 (segment (start 136.868001 75.908001) (end 137.668 76.708) (width 0.25) (layer B.Cu) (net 14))
 (segment (start 136.442999 73.071999) (end 136.442999 75.482999) (width 0.25) (layer B.Cu) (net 14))
 (segment (start 137.378998 72.136) (end 136.442999 73.071999) (width 0.25) (layer B.Cu) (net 14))
 (segment (start 148.988998 72.136) (end 137.378998 72.136) (width 0.25) (layer B.Cu) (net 14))
 (segment (start 132.968001 78.061001) (end 132.043 77.136) (width 0.25) (layer F.Cu) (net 15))
 (segment (start 138.21801 79.79801) (end 136.481001 78.061001) (width 0.25) (layer F.Cu) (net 15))
 (segment (start 157.114541 79.79801) (end 138.21801 79.79801) (width 0.25) (layer F.Cu) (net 15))
 (segment (start 132.043 77.136) (end 130.503 77.136) (width 0.25) (layer F.Cu) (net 15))
 (segment (start 158.60522 78.307329) (end 157.114541 79.79801) (width 0.25) (layer F.Cu) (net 15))
 (segment (start 136.481001 78.061001) (end 132.968001 78.061001) (width 0.25) (layer F.Cu) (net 15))
 (segment (start 158.60522 77.4446) (end 158.60522 78.307329) (width 0.25) (layer F.Cu) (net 15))
 (segment (start 128.787999 76.295999) (end 128.883998 76.2) (width 0.25) (layer F.Cu) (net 16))
 (segment (start 128.787999 79.976001) (end 128.787999 76.295999) (width 0.25) (layer F.Cu) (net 16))
 (segment (start 160.20288 77.4446) (end 160.20288 78.307331) (width 0.25) (layer F.Cu) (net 16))
 (segment (start 160.20288 78.307331) (end 154.4392 84.071011) (width 0.25) (layer F.Cu) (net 16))
 (segment (start 132.883009 84.071011) (end 128.787999 79.976001) (width 0.25) (layer F.Cu) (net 16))
 (segment (start 154.4392 84.071011) (end 132.883009 84.071011) (width 0.25) (layer F.Cu) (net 16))
 (segment (start 133.133 77.136) (end 134.673 77.136) (width 0.25) (layer F.Cu) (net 16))
 (segment (start 132.197 76.2) (end 133.133 77.136) (width 0.25) (layer F.Cu) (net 16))
 (segment (start 128.883998 76.2) (end 132.197 76.2) (width 0.25) (layer F.Cu) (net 16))
 (segment (start 159.40278 78.3296) (end 154.211379 83.521001) (width 0.25) (layer F.Cu) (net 17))
 (segment (start 159.40278 77.4446) (end 159.40278 78.3296) (width 0.25) (layer F.Cu) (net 17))
 (segment (start 130.503 79.886) (end 130.503 79.136) (width 0.25) (layer F.Cu) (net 17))
 (segment (start 130.503 79.992002) (end 130.503 79.886) (width 0.25) (layer F.Cu) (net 17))
 (segment (start 134.031999 83.521001) (end 130.503 79.992002) (width 0.25) (layer F.Cu) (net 17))
 (segment (start 154.211379 83.521001) (end 134.031999 83.521001) (width 0.25) (layer F.Cu) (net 17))
 (segment (start 180.59654 64.516) (end 179.96154 64.516) (width 0.25) (layer F.Cu) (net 18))
 (segment (start 182.206551 66.126011) (end 180.59654 64.516) (width 0.25) (layer F.Cu) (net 18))
 (segment (start 182.206551 70.798822) (end 182.206551 66.126011) (width 0.25) (layer F.Cu) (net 18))
 (segment (start 175.487113 77.51826) (end 182.206551 70.798822) (width 0.25) (layer F.Cu) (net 18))
 (segment (start 161.80308 77.51826) (end 175.487113 77.51826) (width 0.25) (layer F.Cu) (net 18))
 (segment (start 180.59654 67.056) (end 179.96154 67.056) (width 0.25) (layer F.Cu) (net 19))
 (segment (start 181.656541 68.116001) (end 180.59654 67.056) (width 0.25) (layer F.Cu) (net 19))
 (segment (start 181.656541 70.571001) (end 181.656541 68.116001) (width 0.25) (layer F.Cu) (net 19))
 (segment (start 176.276462 75.95108) (end 181.656541 70.571001) (width 0.25) (layer F.Cu) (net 19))
 (segment (start 163.37026 75.95108) (end 176.276462 75.95108) (width 0.25) (layer F.Cu) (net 19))
 (segment (start 183.724999 68.116001) (end 184.785 67.056) (width 0.25) (layer F.Cu) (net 20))
 (segment (start 175.281142 78.502061) (end 183.724999 70.058204) (width 0.25) (layer F.Cu) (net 20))
 (segment (start 161.175441 78.502061) (end 175.281142 78.502061) (width 0.25) (layer F.Cu) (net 20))
 (segment (start 161.00298 78.3296) (end 161.175441 78.502061) (width 0.25) (layer F.Cu) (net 20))
 (segment (start 184.785 67.056) (end 185.42 67.056) (width 0.25) (layer F.Cu) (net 20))
 (segment (start 183.724999 70.058204) (end 183.724999 68.116001) (width 0.25) (layer F.Cu) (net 20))
 (segment (start 161.00298 77.4446) (end 161.00298 78.3296) (width 0.25) (layer F.Cu) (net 20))
 (segment (start 158.60522 60.118798) (end 158.60522 67.9744) (width 0.25) (layer F.Cu) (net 21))
 (segment (start 158.60522 67.9744) (end 158.60522 68.8594) (width 0.25) (layer F.Cu) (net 21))
 (segment (start 165.222831 58.618569) (end 160.105449 58.618569) (width 0.25) (layer F.Cu) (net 21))
 (segment (start 160.105449 58.618569) (end 158.60522 60.118798) (width 0.25) (layer F.Cu) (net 21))
 (segment (start 165.307831 58.703569) (end 165.222831 58.618569) (width 0.25) (layer F.Cu) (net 21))
 (segment (start 175.575178 69.596) (end 165.307831 59.328653) (width 0.25) (layer F.Cu) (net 21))
 (segment (start 165.307831 59.328653) (end 165.307831 58.703569) (width 0.25) (layer F.Cu) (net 21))
 (segment (start 179.96154 69.596) (end 175.575178 69.596) (width 0.25) (layer F.Cu) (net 21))
 (segment (start 172.10786 57.3024) (end 172.10786 57.404) (width 0.25) (layer F.Cu) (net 22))
 (segment (start 171.05903 56.25357) (end 172.10786 57.3024) (width 0.25) (layer F.Cu) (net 22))
 (segment (start 170.95743 56.25357) (end 171.05903 56.25357) (width 0.25) (layer F.Cu) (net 22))
 (segment (start 169.37228 54.66842) (end 170.95743 56.25357) (width 0.25) (layer F.Cu) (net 22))
 (segment (start 169.37228 51.816) (end 169.37228 54.66842) (width 0.25) (layer F.Cu) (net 22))
 (segment (start 161.036 63.0936) (end 164.084 60.0456) (width 0.25) (layer F.Cu) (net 3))
 (segment (start 164.084 60.0456) (end 164.084 59.944) (width 0.25) (layer F.Cu) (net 3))
 (segment (start 161.036 64.008) (end 161.036 63.0936) (width 0.25) (layer F.Cu) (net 3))
 (segment (start 160.20288 67.9744) (end 160.20288 68.8594) (width 0.25) (layer F.Cu) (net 4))
 (segment (start 159.812169 67.583689) (end 160.20288 67.9744) (width 0.25) (layer F.Cu) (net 4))
 (segment (start 159.812169 62.526541) (end 159.812169 67.583689) (width 0.25) (layer F.Cu) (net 4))
 (segment (start 161.24428 61.09443) (end 159.812169 62.526541) (width 0.25) (layer F.Cu) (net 4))
 (segment (start 161.24428 59.944) (end 161.24428 61.09443) (width 0.25) (layer F.Cu) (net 4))
 (segment (start 147.574 52.955) (end 147.574 51.562) (width 0.25) (layer F.Cu) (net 24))
 (segment (start 146.386999 54.142001) (end 147.574 52.955) (width 0.25) (layer F.Cu) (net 24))
 (segment (start 146.386999 59.649001) (end 146.386999 54.142001) (width 0.25) (layer F.Cu) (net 24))
 (segment (start 146.471999 59.734001) (end 146.386999 59.649001) (width 0.25) (layer F.Cu) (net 24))
 (segment (start 149.564721 59.734001) (end 146.471999 59.734001) (width 0.25) (layer F.Cu) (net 24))
 (segment (start 157.80512 67.9744) (end 149.564721 59.734001) (width 0.25) (layer F.Cu) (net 24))
 (segment (start 157.80512 68.8594) (end 157.80512 67.9744) (width 0.25) (layer F.Cu) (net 24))
 (segment (start 136.906 52.955) (end 136.906 51.562) (width 0.25) (layer F.Cu) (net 27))
 (segment (start 135.718999 54.142001) (end 136.906 52.955) (width 0.25) (layer F.Cu) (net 27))
 (segment (start 135.718999 59.649001) (end 135.718999 54.142001) (width 0.25) (layer F.Cu) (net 27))
 (segment (start 149.314631 60.284011) (end 136.354009 60.284011) (width 0.25) (layer F.Cu) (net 27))
 (segment (start 136.354009 60.284011) (end 135.718999 59.649001) (width 0.25) (layer F.Cu) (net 27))
 (segment (start 157.00502 67.9744) (end 149.314631 60.284011) (width 0.25) (layer F.Cu) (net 27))
 (segment (start 157.00502 68.8594) (end 157.00502 67.9744) (width 0.25) (layer F.Cu) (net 27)))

